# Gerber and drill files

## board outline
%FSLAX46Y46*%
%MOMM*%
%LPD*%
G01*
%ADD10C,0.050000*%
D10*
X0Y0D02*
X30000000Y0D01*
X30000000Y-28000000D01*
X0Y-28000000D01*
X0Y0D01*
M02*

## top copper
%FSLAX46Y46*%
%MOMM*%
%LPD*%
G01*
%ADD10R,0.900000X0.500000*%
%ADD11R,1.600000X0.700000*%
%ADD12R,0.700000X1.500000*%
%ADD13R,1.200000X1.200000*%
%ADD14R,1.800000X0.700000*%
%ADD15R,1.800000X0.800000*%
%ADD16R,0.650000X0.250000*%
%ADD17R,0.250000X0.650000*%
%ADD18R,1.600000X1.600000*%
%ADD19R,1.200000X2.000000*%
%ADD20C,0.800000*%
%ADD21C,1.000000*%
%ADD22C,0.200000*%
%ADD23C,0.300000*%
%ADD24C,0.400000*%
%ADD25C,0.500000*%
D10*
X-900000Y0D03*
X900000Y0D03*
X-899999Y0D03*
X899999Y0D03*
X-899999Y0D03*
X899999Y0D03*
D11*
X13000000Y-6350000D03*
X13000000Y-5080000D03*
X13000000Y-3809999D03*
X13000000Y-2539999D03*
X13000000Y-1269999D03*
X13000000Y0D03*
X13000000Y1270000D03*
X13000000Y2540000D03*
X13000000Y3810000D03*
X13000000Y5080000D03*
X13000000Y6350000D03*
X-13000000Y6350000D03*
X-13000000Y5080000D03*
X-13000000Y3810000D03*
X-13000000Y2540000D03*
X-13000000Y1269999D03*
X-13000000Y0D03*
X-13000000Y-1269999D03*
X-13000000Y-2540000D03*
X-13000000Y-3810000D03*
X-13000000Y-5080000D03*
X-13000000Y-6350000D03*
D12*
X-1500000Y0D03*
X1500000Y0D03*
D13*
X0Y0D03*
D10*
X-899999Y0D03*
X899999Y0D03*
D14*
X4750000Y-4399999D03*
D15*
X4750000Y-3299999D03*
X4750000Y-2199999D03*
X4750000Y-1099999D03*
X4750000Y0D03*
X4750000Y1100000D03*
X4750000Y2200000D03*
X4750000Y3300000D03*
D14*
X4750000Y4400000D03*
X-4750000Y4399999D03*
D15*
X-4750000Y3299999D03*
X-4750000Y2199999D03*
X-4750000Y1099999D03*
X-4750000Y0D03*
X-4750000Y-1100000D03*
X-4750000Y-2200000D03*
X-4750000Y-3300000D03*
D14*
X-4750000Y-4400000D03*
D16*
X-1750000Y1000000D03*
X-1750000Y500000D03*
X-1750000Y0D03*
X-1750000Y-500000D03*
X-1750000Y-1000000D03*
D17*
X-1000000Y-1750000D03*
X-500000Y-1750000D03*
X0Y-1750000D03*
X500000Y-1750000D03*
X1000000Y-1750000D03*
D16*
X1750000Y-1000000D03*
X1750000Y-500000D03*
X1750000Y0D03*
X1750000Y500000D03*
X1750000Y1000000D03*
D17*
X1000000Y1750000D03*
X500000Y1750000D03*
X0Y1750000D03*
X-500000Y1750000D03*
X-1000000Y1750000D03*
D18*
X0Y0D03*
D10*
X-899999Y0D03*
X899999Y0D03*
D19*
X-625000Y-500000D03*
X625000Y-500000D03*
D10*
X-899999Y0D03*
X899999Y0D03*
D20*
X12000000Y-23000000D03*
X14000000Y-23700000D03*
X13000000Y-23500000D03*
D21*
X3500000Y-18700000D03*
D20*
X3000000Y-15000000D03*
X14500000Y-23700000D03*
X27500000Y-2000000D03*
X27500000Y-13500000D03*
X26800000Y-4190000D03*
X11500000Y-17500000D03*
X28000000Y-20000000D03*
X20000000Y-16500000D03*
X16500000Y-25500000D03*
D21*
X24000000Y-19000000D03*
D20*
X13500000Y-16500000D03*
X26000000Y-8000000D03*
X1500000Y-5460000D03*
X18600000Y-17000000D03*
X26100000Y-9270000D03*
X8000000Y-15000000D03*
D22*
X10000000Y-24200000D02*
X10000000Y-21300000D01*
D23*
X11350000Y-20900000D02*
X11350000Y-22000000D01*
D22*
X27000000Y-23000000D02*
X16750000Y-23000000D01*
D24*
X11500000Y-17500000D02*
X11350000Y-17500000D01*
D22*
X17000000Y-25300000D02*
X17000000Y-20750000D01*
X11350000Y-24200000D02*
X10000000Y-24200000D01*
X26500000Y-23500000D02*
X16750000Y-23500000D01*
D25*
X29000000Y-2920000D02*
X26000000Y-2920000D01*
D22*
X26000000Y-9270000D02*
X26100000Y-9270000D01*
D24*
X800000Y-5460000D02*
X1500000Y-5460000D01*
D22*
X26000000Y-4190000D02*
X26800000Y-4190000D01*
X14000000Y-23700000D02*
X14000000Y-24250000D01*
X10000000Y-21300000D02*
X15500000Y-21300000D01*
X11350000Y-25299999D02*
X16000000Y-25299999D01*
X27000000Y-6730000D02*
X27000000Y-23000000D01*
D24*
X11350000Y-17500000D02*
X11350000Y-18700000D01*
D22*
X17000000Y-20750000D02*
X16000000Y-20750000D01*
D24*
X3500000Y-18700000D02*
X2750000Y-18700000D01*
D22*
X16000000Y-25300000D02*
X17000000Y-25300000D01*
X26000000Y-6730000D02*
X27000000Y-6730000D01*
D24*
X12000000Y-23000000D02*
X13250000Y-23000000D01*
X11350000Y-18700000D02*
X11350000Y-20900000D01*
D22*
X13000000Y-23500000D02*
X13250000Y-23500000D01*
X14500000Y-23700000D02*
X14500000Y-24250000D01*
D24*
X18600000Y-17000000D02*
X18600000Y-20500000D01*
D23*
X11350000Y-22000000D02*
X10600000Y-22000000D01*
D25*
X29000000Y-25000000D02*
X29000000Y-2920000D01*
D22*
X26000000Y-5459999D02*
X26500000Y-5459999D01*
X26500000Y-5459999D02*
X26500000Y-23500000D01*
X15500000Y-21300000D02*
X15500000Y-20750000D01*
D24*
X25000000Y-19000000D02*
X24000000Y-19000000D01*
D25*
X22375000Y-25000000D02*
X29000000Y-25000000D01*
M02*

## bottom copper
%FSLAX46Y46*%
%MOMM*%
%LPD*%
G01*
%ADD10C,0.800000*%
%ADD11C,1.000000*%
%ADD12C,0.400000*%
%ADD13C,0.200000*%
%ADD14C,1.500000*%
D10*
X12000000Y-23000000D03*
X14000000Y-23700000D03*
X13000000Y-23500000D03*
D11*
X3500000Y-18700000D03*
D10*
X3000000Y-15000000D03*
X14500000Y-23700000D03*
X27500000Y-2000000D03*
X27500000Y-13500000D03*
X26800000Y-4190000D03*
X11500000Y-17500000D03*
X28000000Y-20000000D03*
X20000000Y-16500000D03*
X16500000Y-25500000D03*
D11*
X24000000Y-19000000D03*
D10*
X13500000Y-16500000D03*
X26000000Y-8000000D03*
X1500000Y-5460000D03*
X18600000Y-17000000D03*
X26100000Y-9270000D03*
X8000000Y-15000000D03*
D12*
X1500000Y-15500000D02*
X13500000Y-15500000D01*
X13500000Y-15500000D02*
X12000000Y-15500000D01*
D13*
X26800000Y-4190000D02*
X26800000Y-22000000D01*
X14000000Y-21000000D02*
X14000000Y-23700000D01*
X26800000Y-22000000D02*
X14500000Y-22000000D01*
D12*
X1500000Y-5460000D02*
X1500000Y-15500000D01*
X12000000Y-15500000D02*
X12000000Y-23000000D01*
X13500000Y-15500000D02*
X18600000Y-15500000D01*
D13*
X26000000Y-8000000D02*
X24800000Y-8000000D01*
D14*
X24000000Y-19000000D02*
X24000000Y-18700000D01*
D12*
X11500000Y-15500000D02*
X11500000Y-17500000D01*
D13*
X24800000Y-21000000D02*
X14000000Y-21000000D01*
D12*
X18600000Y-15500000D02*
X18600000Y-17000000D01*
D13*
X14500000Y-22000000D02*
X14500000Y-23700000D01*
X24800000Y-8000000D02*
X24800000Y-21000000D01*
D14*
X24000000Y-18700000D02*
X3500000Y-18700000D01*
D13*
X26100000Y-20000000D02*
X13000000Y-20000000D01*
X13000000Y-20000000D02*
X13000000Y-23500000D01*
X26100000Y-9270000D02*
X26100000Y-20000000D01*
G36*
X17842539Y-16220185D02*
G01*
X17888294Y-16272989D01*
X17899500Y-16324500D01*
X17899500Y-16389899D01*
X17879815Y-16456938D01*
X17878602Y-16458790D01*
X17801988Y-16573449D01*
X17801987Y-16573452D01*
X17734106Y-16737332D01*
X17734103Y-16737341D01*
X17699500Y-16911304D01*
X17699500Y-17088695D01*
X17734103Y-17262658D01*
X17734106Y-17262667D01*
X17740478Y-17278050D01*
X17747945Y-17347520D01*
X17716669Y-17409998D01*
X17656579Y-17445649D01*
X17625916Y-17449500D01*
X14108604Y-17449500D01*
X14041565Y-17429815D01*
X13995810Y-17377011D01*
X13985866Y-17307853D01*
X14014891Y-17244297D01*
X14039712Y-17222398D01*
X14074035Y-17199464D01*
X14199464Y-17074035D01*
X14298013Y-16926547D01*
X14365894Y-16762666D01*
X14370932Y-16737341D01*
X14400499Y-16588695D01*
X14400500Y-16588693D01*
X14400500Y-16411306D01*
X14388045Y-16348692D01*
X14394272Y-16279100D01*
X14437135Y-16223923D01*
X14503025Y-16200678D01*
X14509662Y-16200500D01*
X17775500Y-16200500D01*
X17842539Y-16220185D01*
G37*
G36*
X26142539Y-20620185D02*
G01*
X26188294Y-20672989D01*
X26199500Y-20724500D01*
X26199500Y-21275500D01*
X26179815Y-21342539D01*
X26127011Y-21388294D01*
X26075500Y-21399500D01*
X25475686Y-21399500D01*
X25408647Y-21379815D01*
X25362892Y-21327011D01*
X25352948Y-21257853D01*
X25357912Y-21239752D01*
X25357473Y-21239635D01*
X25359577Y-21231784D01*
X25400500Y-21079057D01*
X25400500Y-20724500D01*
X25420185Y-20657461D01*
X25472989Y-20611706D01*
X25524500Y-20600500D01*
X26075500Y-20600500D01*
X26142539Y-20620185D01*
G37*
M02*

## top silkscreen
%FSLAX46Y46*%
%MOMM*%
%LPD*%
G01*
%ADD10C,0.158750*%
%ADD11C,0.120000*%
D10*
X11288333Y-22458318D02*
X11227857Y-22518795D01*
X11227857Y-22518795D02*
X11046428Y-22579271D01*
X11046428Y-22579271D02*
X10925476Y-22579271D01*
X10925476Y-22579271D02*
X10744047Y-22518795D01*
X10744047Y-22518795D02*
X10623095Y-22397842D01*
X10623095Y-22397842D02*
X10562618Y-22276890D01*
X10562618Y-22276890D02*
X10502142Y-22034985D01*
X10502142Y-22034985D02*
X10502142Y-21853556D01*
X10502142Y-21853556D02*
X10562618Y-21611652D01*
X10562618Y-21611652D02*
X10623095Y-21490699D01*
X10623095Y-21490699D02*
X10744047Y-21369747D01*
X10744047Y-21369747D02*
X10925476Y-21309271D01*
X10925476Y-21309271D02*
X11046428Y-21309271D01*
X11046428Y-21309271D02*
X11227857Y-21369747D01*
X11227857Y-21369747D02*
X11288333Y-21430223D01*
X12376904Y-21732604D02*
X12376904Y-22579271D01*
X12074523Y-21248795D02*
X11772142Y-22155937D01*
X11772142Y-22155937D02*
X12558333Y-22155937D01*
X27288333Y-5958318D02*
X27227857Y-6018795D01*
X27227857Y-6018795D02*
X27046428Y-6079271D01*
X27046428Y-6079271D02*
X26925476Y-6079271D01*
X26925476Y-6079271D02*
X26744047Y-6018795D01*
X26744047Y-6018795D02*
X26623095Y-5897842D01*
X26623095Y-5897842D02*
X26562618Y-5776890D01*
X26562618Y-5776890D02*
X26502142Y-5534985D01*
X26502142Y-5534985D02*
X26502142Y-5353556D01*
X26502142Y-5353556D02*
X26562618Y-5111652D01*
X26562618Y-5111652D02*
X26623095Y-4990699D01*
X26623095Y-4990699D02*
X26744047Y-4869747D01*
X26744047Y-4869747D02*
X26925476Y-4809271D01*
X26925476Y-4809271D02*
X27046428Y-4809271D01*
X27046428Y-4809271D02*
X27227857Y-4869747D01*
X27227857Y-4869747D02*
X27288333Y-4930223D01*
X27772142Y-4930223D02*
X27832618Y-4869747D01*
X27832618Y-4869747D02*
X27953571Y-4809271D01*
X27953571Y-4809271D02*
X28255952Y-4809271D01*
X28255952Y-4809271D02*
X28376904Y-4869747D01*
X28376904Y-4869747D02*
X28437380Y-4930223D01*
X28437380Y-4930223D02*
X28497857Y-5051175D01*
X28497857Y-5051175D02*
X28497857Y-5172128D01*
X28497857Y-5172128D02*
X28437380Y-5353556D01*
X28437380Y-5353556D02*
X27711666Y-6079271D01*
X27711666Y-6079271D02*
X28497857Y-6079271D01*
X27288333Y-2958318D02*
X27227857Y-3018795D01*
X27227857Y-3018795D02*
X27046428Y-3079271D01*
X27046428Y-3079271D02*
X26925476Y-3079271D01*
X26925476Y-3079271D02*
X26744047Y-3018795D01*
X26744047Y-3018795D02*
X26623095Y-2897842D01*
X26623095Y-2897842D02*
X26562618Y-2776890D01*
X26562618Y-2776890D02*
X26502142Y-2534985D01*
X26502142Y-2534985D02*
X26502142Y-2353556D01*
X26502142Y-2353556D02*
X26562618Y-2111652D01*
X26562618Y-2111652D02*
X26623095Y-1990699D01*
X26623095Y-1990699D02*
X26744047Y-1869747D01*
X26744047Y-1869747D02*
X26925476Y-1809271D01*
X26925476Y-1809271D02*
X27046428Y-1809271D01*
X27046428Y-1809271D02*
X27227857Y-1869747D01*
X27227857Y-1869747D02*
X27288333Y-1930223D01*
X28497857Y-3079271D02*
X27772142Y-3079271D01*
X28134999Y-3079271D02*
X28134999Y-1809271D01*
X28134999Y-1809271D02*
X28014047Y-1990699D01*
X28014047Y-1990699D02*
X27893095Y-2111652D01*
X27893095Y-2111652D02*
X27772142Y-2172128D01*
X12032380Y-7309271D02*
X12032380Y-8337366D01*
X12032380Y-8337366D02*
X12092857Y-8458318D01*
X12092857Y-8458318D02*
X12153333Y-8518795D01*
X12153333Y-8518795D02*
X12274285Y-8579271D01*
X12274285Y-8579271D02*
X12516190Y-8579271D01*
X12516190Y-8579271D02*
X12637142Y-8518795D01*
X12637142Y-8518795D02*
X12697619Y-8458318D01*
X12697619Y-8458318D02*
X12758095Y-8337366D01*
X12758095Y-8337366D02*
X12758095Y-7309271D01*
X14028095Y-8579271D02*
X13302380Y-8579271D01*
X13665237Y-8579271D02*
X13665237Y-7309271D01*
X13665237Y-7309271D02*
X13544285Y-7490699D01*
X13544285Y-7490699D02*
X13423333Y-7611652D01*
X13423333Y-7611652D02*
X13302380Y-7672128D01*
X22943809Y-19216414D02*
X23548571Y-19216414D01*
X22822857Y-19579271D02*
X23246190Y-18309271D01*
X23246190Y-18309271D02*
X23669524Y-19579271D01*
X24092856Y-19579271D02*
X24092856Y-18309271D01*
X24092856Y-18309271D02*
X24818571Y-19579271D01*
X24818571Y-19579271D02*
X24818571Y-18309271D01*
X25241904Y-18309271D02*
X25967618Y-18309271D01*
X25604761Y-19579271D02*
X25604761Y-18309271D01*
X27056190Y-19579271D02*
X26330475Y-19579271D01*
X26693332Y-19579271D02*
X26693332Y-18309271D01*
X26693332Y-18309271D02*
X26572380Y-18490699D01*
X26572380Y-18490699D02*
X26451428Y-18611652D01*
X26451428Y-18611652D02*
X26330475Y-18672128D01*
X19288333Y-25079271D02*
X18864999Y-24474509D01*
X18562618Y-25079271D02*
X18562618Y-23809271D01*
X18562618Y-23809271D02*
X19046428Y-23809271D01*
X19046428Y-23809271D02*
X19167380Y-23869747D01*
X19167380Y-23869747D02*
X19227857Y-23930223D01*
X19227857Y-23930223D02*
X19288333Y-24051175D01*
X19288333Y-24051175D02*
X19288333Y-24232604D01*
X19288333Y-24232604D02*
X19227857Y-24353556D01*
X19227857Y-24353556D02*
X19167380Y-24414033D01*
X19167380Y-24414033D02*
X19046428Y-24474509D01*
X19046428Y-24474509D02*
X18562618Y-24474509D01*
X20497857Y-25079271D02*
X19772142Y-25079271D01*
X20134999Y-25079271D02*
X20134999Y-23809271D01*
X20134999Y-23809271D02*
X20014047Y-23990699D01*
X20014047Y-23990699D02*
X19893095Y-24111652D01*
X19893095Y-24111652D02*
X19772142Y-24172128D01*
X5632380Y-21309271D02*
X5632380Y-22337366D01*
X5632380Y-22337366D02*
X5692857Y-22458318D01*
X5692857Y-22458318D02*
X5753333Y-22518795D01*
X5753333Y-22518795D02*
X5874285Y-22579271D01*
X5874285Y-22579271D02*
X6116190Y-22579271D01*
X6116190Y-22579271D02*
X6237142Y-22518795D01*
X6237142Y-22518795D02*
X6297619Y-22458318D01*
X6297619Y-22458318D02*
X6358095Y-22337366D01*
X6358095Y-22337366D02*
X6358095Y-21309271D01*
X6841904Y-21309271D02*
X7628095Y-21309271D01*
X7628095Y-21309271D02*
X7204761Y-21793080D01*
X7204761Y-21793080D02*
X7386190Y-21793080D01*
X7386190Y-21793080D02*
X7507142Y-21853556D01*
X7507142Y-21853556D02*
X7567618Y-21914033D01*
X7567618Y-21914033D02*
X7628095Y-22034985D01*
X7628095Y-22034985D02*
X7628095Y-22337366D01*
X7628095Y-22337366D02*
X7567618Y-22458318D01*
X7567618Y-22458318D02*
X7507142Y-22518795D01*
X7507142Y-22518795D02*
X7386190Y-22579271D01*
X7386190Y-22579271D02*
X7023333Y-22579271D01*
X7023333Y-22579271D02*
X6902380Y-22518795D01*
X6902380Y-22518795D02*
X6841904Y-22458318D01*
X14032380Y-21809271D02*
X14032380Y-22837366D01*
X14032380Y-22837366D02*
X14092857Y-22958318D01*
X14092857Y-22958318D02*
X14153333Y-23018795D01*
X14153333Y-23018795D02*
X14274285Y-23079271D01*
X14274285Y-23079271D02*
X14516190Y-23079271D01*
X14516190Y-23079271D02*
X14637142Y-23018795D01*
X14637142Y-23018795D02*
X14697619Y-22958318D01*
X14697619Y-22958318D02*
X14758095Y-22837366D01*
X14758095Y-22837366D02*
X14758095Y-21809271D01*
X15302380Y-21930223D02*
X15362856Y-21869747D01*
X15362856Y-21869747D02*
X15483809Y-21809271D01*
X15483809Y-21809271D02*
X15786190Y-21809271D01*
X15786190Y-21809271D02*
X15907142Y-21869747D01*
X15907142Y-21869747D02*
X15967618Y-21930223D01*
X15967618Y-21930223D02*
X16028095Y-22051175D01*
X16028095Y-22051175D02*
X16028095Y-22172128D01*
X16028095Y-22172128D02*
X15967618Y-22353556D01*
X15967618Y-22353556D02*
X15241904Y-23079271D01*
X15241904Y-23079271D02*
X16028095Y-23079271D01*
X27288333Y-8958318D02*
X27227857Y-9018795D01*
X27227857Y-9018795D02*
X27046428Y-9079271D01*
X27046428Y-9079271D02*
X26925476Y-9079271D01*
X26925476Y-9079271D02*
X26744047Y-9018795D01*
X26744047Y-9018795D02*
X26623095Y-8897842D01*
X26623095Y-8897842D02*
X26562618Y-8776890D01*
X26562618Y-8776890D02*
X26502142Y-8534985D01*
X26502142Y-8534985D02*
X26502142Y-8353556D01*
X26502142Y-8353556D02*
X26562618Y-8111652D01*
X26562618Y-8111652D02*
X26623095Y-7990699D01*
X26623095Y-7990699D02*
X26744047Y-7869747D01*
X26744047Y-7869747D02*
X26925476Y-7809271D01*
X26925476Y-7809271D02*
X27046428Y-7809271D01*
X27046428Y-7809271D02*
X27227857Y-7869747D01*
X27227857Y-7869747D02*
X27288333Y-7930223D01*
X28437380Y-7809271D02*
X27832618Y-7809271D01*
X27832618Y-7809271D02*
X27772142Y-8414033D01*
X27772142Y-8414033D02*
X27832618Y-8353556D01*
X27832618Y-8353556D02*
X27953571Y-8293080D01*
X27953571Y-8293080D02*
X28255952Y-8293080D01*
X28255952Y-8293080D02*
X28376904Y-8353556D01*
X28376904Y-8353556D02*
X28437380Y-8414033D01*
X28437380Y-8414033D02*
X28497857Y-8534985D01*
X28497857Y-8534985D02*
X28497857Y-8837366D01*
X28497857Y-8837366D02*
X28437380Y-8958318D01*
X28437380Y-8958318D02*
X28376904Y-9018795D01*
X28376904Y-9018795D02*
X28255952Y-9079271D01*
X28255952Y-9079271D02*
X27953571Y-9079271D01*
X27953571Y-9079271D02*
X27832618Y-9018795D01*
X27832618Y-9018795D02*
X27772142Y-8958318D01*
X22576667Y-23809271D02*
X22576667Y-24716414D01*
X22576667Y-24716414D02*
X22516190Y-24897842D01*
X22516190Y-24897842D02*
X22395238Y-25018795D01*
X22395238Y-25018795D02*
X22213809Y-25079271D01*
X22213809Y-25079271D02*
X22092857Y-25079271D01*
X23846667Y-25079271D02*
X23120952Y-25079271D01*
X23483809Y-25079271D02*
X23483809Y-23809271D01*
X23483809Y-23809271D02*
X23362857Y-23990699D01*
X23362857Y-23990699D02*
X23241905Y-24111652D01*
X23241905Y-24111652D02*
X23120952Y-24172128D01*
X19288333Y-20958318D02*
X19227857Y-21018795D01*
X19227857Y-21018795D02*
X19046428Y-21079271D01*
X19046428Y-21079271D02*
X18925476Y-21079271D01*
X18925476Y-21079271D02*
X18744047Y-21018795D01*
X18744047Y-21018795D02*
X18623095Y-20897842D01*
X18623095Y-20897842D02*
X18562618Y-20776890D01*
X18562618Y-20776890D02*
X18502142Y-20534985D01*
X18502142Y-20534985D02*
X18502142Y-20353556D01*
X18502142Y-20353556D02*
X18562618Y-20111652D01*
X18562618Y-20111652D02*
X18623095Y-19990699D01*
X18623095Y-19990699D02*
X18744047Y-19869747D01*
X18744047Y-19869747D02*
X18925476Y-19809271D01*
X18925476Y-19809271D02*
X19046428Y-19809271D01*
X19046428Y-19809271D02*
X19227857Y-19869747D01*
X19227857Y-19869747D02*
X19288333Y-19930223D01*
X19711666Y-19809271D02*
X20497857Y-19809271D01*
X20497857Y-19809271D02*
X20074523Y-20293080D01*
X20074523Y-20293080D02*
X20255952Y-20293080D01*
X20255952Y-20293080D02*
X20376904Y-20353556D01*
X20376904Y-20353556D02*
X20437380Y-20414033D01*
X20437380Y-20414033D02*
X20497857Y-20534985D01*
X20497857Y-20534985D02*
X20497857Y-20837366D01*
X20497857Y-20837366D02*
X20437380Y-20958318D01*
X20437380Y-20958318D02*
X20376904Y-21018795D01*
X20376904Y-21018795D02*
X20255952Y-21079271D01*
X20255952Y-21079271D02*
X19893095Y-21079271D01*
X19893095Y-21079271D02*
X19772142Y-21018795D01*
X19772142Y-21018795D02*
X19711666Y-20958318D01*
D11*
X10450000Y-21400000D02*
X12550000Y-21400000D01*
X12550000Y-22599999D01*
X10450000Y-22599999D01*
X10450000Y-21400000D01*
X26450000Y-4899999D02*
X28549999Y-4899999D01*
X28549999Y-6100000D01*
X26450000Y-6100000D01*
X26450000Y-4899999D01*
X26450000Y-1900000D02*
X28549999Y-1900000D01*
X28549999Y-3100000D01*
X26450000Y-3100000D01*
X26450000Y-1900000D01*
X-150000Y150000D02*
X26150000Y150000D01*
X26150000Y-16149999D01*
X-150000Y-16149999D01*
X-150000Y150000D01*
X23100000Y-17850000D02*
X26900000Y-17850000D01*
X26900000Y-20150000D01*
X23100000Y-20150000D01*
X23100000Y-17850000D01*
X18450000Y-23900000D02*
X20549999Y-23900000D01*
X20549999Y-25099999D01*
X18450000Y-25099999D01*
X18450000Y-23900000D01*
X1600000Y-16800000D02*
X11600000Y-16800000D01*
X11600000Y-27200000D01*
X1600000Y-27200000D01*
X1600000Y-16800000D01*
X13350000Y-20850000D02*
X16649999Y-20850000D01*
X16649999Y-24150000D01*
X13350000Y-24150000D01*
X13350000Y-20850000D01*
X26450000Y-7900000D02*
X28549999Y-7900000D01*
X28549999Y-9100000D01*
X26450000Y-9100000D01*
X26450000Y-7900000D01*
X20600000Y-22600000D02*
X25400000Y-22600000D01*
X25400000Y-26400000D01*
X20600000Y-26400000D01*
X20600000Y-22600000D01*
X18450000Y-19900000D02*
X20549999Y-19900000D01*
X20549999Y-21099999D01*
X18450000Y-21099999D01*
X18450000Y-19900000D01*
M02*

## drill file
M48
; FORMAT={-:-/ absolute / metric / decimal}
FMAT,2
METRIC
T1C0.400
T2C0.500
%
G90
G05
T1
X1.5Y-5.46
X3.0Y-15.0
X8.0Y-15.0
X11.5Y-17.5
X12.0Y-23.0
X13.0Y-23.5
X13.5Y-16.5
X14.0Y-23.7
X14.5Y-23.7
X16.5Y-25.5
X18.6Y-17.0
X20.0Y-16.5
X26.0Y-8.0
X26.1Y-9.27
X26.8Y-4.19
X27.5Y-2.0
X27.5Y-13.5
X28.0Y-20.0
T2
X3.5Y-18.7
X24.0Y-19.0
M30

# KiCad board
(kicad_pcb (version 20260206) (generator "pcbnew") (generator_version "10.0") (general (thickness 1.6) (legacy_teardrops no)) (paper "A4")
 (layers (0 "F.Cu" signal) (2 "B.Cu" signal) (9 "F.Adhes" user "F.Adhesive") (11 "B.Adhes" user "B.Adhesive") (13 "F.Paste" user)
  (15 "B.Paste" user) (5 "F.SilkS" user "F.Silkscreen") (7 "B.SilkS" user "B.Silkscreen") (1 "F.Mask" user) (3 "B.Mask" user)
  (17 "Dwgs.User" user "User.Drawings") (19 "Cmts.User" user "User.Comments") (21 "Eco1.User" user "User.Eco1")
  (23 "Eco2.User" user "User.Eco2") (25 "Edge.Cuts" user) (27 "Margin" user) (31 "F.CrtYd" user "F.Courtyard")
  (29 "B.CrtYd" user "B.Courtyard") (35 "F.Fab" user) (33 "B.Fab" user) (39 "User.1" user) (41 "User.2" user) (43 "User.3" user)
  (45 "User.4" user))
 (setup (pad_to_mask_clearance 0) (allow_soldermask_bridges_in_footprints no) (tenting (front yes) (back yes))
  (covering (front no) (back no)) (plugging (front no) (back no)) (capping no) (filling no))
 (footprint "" (layer "F.Cu") (at 11.5 22)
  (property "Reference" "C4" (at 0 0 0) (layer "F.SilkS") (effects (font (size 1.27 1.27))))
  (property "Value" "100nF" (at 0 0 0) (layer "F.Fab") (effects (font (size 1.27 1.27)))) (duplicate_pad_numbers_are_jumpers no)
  (fp_rect (start -1.05 -0.6) (end 1.05 0.599999) (stroke (width 0.12) (type default)) (fill no) (layer "F.SilkS"))
  (pad "1" smd rect (at -12.4 -22) (size 0.9 0.5) (layers "F.Cu" "F.Mask" "F.Paste") (thermal_bridge_angle 45))
  (pad "2" smd rect (at -10.6 -22) (size 0.9 0.5) (layers "F.Cu" "F.Mask" "F.Paste") (thermal_bridge_angle 45)))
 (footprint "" (layer "F.Cu") (at 27.5 5.5)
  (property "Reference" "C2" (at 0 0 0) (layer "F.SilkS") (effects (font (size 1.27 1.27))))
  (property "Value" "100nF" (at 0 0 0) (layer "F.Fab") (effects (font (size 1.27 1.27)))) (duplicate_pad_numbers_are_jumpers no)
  (fp_rect (start -1.05 -0.600001) (end 1.049999 0.6) (stroke (width 0.12) (type default)) (fill no) (layer "F.SilkS"))
  (pad "1" smd rect (at -28.399999 -5.5) (size 0.9 0.5) (layers "F.Cu" "F.Mask" "F.Paste") (thermal_bridge_angle 45))
  (pad "2" smd rect (at -26.600001 -5.5) (size 0.9 0.5) (layers "F.Cu" "F.Mask" "F.Paste") (thermal_bridge_angle 45)))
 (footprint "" (layer "F.Cu") (at 27.5 2.5)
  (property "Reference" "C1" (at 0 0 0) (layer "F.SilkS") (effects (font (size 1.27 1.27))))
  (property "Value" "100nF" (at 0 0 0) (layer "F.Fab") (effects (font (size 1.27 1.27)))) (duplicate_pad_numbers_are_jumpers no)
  (fp_rect (start -1.05 -0.6) (end 1.049999 0.6) (stroke (width 0.12) (type default)) (fill no) (layer "F.SilkS"))
  (pad "1" smd rect (at -28.399999 -2.5) (size 0.9 0.5) (layers "F.Cu" "F.Mask" "F.Paste") (thermal_bridge_angle 45))
  (pad "2" smd rect (at -26.600001 -2.5) (size 0.9 0.5) (layers "F.Cu" "F.Mask" "F.Paste") (thermal_bridge_angle 45)))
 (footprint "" (layer "F.Cu") (at 13 8)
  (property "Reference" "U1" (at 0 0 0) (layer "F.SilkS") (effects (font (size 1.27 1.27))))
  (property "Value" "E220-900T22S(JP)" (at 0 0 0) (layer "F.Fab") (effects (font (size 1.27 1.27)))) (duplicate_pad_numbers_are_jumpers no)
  (fp_rect (start -13.15 -8.15) (end 13.15 8.149999) (stroke (width 0.12) (type default)) (fill no) (layer "F.SilkS"))
  (pad "1" smd rect (at 0 -1.65) (size 1.6 0.7) (layers "F.Cu" "F.Mask" "F.Paste") (thermal_bridge_angle 45))
  (pad "2" smd rect (at 0 -2.92) (size 1.6 0.7) (layers "F.Cu" "F.Mask" "F.Paste") (thermal_bridge_angle 45))
  (pad "3" smd rect (at 0 -4.190001) (size 1.6 0.7) (layers "F.Cu" "F.Mask" "F.Paste") (thermal_bridge_angle 45))
  (pad "4" smd rect (at 0 -5.460001) (size 1.6 0.7) (layers "F.Cu" "F.Mask" "F.Paste") (thermal_bridge_angle 45))
  (pad "5" smd rect (at 0 -6.730001) (size 1.6 0.7) (layers "F.Cu" "F.Mask" "F.Paste") (thermal_bridge_angle 45))
  (pad "6" smd rect (at 0 -8) (size 1.6 0.7) (layers "F.Cu" "F.Mask" "F.Paste") (thermal_bridge_angle 45))
  (pad "7" smd rect (at 0 -9.27) (size 1.6 0.7) (layers "F.Cu" "F.Mask" "F.Paste") (thermal_bridge_angle 45))
  (pad "8" smd rect (at 0 -10.54) (size 1.6 0.7) (layers "F.Cu" "F.Mask" "F.Paste") (thermal_bridge_angle 45))
  (pad "9" smd rect (at 0 -11.81) (size 1.6 0.7) (layers "F.Cu" "F.Mask" "F.Paste") (thermal_bridge_angle 45))
  (pad "10" smd rect (at 0 -13.08) (size 1.6 0.7) (layers "F.Cu" "F.Mask" "F.Paste") (thermal_bridge_angle 45))
  (pad "11" smd rect (at 0 -14.35) (size 1.6 0.7) (layers "F.Cu" "F.Mask" "F.Paste") (thermal_bridge_angle 45))
  (pad "12" smd rect (at -26 -14.35) (size 1.6 0.7) (layers "F.Cu" "F.Mask" "F.Paste") (thermal_bridge_angle 45))
  (pad "13" smd rect (at -26 -13.08) (size 1.6 0.7) (layers "F.Cu" "F.Mask" "F.Paste") (thermal_bridge_angle 45))
  (pad "14" smd rect (at -26 -11.81) (size 1.6 0.7) (layers "F.Cu" "F.Mask" "F.Paste") (thermal_bridge_angle 45))
  (pad "15" smd rect (at -26 -10.54) (size 1.6 0.7) (layers "F.Cu" "F.Mask" "F.Paste") (thermal_bridge_angle 45))
  (pad "16" smd rect (at -26 -9.269999) (size 1.6 0.7) (layers "F.Cu" "F.Mask" "F.Paste") (thermal_bridge_angle 45))
  (pad "17" smd rect (at -26 -8) (size 1.6 0.7) (layers "F.Cu" "F.Mask" "F.Paste") (thermal_bridge_angle 45))
  (pad "18" smd rect (at -26 -6.730001) (size 1.6 0.7) (layers "F.Cu" "F.Mask" "F.Paste") (thermal_bridge_angle 45))
  (pad "19" smd rect (at -26 -5.46) (size 1.6 0.7) (layers "F.Cu" "F.Mask" "F.Paste") (thermal_bridge_angle 45))
  (pad "20" smd rect (at -26 -4.19) (size 1.6 0.7) (layers "F.Cu" "F.Mask" "F.Paste") (thermal_bridge_angle 45))
  (pad "21" smd rect (at -26 -2.92) (size 1.6 0.7) (layers "F.Cu" "F.Mask" "F.Paste") (thermal_bridge_angle 45))
  (pad "22" smd rect (at -26 -1.65) (size 1.6 0.7) (layers "F.Cu" "F.Mask" "F.Paste") (thermal_bridge_angle 45)))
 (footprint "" (layer "F.Cu") (at 25 19)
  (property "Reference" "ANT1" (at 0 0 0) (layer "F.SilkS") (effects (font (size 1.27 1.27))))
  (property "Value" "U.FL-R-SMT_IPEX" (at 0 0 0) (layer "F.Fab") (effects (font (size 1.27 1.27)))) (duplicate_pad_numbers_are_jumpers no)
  (fp_rect (start -1.9 -1.15) (end 1.9 1.15) (stroke (width 0.12) (type default)) (fill no) (layer "F.SilkS"))
  (pad "G1" smd rect (at -26.5 -19) (size 0.7 1.5) (layers "F.Cu" "F.Mask" "F.Paste") (thermal_bridge_angle 45))
  (pad "G2" smd rect (at -23.5 -19) (size 0.7 1.5) (layers "F.Cu" "F.Mask" "F.Paste") (thermal_bridge_angle 45))
  (pad "S" smd rect (at -25 -19) (size 1.2 1.2) (layers "F.Cu" "F.Mask" "F.Paste") (thermal_bridge_angle 45)))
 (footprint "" (layer "F.Cu") (at 19.5 24.5)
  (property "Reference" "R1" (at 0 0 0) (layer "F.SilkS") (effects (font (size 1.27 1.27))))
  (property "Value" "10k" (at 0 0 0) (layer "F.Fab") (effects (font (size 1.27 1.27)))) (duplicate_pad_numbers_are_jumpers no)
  (fp_rect (start -1.05 -0.6) (end 1.049999 0.599999) (stroke (width 0.12) (type default)) (fill no) (layer "F.SilkS"))
  (pad "1" smd rect (at -20.399999 -24.5) (size 0.9 0.5) (layers "F.Cu" "F.Mask" "F.Paste") (thermal_bridge_angle 45))
  (pad "2" smd rect (at -18.600001 -24.5) (size 0.9 0.5) (layers "F.Cu" "F.Mask" "F.Paste") (thermal_bridge_angle 45)))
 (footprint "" (layer "F.Cu") (at 6.6 22)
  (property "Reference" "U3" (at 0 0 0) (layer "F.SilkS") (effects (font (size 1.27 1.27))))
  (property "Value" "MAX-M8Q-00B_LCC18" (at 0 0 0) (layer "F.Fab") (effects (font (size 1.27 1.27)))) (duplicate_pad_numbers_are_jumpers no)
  (fp_rect (start -5 -5.2) (end 5 5.2) (stroke (width 0.12) (type default)) (fill no) (layer "F.SilkS"))
  (pad "1" smd rect (at -1.85 -17.600001) (size 1.8 0.7) (layers "F.Cu" "F.Mask" "F.Paste") (thermal_bridge_angle 45))
  (pad "2" smd rect (at -1.85 -18.700001) (size 1.8 0.8) (layers "F.Cu" "F.Mask" "F.Paste") (thermal_bridge_angle 45))
  (pad "3" smd rect (at -1.85 -19.800001) (size 1.8 0.8) (layers "F.Cu" "F.Mask" "F.Paste") (thermal_bridge_angle 45))
  (pad "4" smd rect (at -1.85 -20.900001) (size 1.8 0.8) (layers "F.Cu" "F.Mask" "F.Paste") (thermal_bridge_angle 45))
  (pad "5" smd rect (at -1.85 -22) (size 1.8 0.8) (layers "F.Cu" "F.Mask" "F.Paste") (thermal_bridge_angle 45))
  (pad "6" smd rect (at -1.85 -23.1) (size 1.8 0.8) (layers "F.Cu" "F.Mask" "F.Paste") (thermal_bridge_angle 45))
  (pad "7" smd rect (at -1.85 -24.2) (size 1.8 0.8) (layers "F.Cu" "F.Mask" "F.Paste") (thermal_bridge_angle 45))
  (pad "8" smd rect (at -1.85 -25.3) (size 1.8 0.8) (layers "F.Cu" "F.Mask" "F.Paste") (thermal_bridge_angle 45))
  (pad "9" smd rect (at -1.85 -26.4) (size 1.8 0.7) (layers "F.Cu" "F.Mask" "F.Paste") (thermal_bridge_angle 45))
  (pad "10" smd rect (at -11.35 -26.399999) (size 1.8 0.7) (layers "F.Cu" "F.Mask" "F.Paste") (thermal_bridge_angle 45))
  (pad "11" smd rect (at -11.35 -25.299999) (size 1.8 0.8) (layers "F.Cu" "F.Mask" "F.Paste") (thermal_bridge_angle 45))
  (pad "12" smd rect (at -11.35 -24.199999) (size 1.8 0.8) (layers "F.Cu" "F.Mask" "F.Paste") (thermal_bridge_angle 45))
  (pad "13" smd rect (at -11.35 -23.099999) (size 1.8 0.8) (layers "F.Cu" "F.Mask" "F.Paste") (thermal_bridge_angle 45))
  (pad "14" smd rect (at -11.35 -22) (size 1.8 0.8) (layers "F.Cu" "F.Mask" "F.Paste") (thermal_bridge_angle 45))
  (pad "15" smd rect (at -11.35 -20.9) (size 1.8 0.8) (layers "F.Cu" "F.Mask" "F.Paste") (thermal_bridge_angle 45))
  (pad "16" smd rect (at -11.35 -19.8) (size 1.8 0.8) (layers "F.Cu" "F.Mask" "F.Paste") (thermal_bridge_angle 45))
  (pad "17" smd rect (at -11.35 -18.7) (size 1.8 0.8) (layers "F.Cu" "F.Mask" "F.Paste") (thermal_bridge_angle 45))
  (pad "18" smd rect (at -11.35 -17.6) (size 1.8 0.7) (layers "F.Cu" "F.Mask" "F.Paste") (thermal_bridge_angle 45)))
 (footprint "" (layer "F.Cu") (at 15 22.5)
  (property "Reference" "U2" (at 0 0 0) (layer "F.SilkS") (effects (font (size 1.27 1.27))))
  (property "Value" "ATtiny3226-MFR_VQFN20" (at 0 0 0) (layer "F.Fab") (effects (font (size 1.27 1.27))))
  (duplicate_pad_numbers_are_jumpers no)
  (fp_rect (start -1.65 -1.65) (end 1.649999 1.65) (stroke (width 0.12) (type default)) (fill no) (layer "F.SilkS"))
  (pad "1" smd rect (at -16.75 -23.5) (size 0.65 0.25) (layers "F.Cu" "F.Mask" "F.Paste") (thermal_bridge_angle 45))
  (pad "2" smd rect (at -16.75 -23) (size 0.65 0.25) (layers "F.Cu" "F.Mask" "F.Paste") (thermal_bridge_angle 45))
  (pad "3" smd rect (at -16.75 -22.5) (size 0.65 0.25) (layers "F.Cu" "F.Mask" "F.Paste") (thermal_bridge_angle 45))
  (pad "4" smd rect (at -16.75 -22) (size 0.65 0.25) (layers "F.Cu" "F.Mask" "F.Paste") (thermal_bridge_angle 45))
  (pad "5" smd rect (at -16.75 -21.5) (size 0.65 0.25) (layers "F.Cu" "F.Mask" "F.Paste") (thermal_bridge_angle 45))
  (pad "6" smd rect (at -16 -20.75) (size 0.25 0.65) (layers "F.Cu" "F.Mask" "F.Paste") (thermal_bridge_angle 45))
  (pad "7" smd rect (at -15.5 -20.75) (size 0.25 0.65) (layers "F.Cu" "F.Mask" "F.Paste") (thermal_bridge_angle 45))
  (pad "8" smd rect (at -15 -20.75) (size 0.25 0.65) (layers "F.Cu" "F.Mask" "F.Paste") (thermal_bridge_angle 45))
  (pad "9" smd rect (at -14.5 -20.75) (size 0.25 0.65) (layers "F.Cu" "F.Mask" "F.Paste") (thermal_bridge_angle 45))
  (pad "10" smd rect (at -14 -20.75) (size 0.25 0.65) (layers "F.Cu" "F.Mask" "F.Paste") (thermal_bridge_angle 45))
  (pad "11" smd rect (at -13.25 -21.5) (size 0.65 0.25) (layers "F.Cu" "F.Mask" "F.Paste") (thermal_bridge_angle 45))
  (pad "12" smd rect (at -13.25 -22) (size 0.65 0.25) (layers "F.Cu" "F.Mask" "F.Paste") (thermal_bridge_angle 45))
  (pad "13" smd rect (at -13.25 -22.5) (size 0.65 0.25) (layers "F.Cu" "F.Mask" "F.Paste") (thermal_bridge_angle 45))
  (pad "14" smd rect (at -13.25 -23) (size 0.65 0.25) (layers "F.Cu" "F.Mask" "F.Paste") (thermal_bridge_angle 45))
  (pad "15" smd rect (at -13.25 -23.5) (size 0.65 0.25) (layers "F.Cu" "F.Mask" "F.Paste") (thermal_bridge_angle 45))
  (pad "16" smd rect (at -14 -24.25) (size 0.25 0.65) (layers "F.Cu" "F.Mask" "F.Paste") (thermal_bridge_angle 45))
  (pad "17" smd rect (at -14.5 -24.25) (size 0.25 0.65) (layers "F.Cu" "F.Mask" "F.Paste") (thermal_bridge_angle 45))
  (pad "18" smd rect (at -15 -24.25) (size 0.25 0.65) (layers "F.Cu" "F.Mask" "F.Paste") (thermal_bridge_angle 45))
  (pad "19" smd rect (at -15.5 -24.25) (size 0.25 0.65) (layers "F.Cu" "F.Mask" "F.Paste") (thermal_bridge_angle 45))
  (pad "20" smd rect (at -16 -24.25) (size 0.25 0.65) (layers "F.Cu" "F.Mask" "F.Paste") (thermal_bridge_angle 45))
  (pad "EP" smd rect (at -15 -22.5) (size 1.6 1.6) (layers "F.Cu" "F.Mask" "F.Paste") (thermal_bridge_angle 45)))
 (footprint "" (layer "F.Cu") (at 27.5 8.5)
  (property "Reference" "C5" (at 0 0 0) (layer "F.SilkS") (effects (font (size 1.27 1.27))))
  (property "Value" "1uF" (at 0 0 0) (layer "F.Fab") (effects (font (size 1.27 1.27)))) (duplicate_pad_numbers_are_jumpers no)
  (fp_rect (start -1.05 -0.6) (end 1.049999 0.6) (stroke (width 0.12) (type default)) (fill no) (layer "F.SilkS"))
  (pad "1" smd rect (at -28.399999 -8.5) (size 0.9 0.5) (layers "F.Cu" "F.Mask" "F.Paste") (thermal_bridge_angle 45))
  (pad "2" smd rect (at -26.600001 -8.5) (size 0.9 0.5) (layers "F.Cu" "F.Mask" "F.Paste") (thermal_bridge_angle 45)))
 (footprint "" (layer "F.Cu") (at 23 24.5)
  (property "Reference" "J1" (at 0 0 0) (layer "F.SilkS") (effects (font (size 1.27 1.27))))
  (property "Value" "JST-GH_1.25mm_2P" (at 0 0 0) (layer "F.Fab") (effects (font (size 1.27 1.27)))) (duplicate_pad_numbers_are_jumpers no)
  (fp_rect (start -2.4 -1.9) (end 2.4 1.9) (stroke (width 0.12) (type default)) (fill no) (layer "F.SilkS"))
  (pad "1" smd rect (at -23.625 -24) (size 1.2 2) (layers "F.Cu" "F.Mask" "F.Paste") (thermal_bridge_angle 45))
  (pad "2" smd rect (at -22.375 -24) (size 1.2 2) (layers "F.Cu" "F.Mask" "F.Paste") (thermal_bridge_angle 45)))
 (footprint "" (layer "F.Cu") (at 19.5 20.5)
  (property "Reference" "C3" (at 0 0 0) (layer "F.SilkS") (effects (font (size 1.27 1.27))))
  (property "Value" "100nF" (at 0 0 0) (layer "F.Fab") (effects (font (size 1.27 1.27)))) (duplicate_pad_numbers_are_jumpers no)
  (fp_rect (start -1.05 -0.6) (end 1.049999 0.599999) (stroke (width 0.12) (type default)) (fill no) (layer "F.SilkS"))
  (pad "1" smd rect (at -20.399999 -20.5) (size 0.9 0.5) (layers "F.Cu" "F.Mask" "F.Paste") (thermal_bridge_angle 45))
  (pad "2" smd rect (at -18.600001 -20.5) (size 0.9 0.5) (layers "F.Cu" "F.Mask" "F.Paste") (thermal_bridge_angle 45)))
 (gr_rect (start 0 0) (end 30 28) (stroke (width 0.05) (type default)) (fill no) (layer "Edge.Cuts"))
 (segment (start 10 24.2) (end 10 21.3) (width 0.2) (layer "F.Cu") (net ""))
 (segment (start 11.35 20.9) (end 11.35 22) (width 0.3) (layer "F.Cu") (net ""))
 (segment (start 27 23) (end 16.75 23) (width 0.2) (layer "F.Cu") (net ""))
 (segment (start 11.5 17.5) (end 11.35 17.5) (width 0.4) (layer "F.Cu") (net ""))
 (segment (start 17 25.3) (end 17 20.75) (width 0.2) (layer "F.Cu") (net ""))
 (segment (start 11.35 24.2) (end 10 24.2) (width 0.2) (layer "F.Cu") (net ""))
 (segment (start 26.5 23.5) (end 16.75 23.5) (width 0.2) (layer "F.Cu") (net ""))
 (segment (start 29 2.92) (end 26 2.92) (width 0.5) (layer "F.Cu") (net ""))
 (segment (start 26 9.27) (end 26.1 9.27) (width 0.2) (layer "F.Cu") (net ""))
 (segment (start 0.8 5.46) (end 1.5 5.46) (width 0.4) (layer "F.Cu") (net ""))
 (segment (start 26 4.19) (end 26.8 4.19) (width 0.2) (layer "F.Cu") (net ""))
 (segment (start 14 23.7) (end 14 24.25) (width 0.2) (layer "F.Cu") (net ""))
 (segment (start 10 21.3) (end 15.5 21.3) (width 0.2) (layer "F.Cu") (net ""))
 (segment (start 11.35 25.299999) (end 16 25.299999) (width 0.2) (layer "F.Cu") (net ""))
 (segment (start 27 6.73) (end 27 23) (width 0.2) (layer "F.Cu") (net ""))
 (segment (start 11.35 17.5) (end 11.35 18.7) (width 0.4) (layer "F.Cu") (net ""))
 (segment (start 17 20.75) (end 16 20.75) (width 0.2) (layer "F.Cu") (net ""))
 (segment (start 3.5 18.7) (end 2.75 18.7) (width 0.4) (layer "F.Cu") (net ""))
 (segment (start 16 25.3) (end 17 25.3) (width 0.2) (layer "F.Cu") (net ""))
 (segment (start 26 6.73) (end 27 6.73) (width 0.2) (layer "F.Cu") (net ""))
 (segment (start 12 23) (end 13.25 23) (width 0.4) (layer "F.Cu") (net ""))
 (segment (start 11.35 18.7) (end 11.35 20.9) (width 0.4) (layer "F.Cu") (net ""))
 (segment (start 13 23.5) (end 13.25 23.5) (width 0.2) (layer "F.Cu") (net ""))
 (segment (start 14.5 23.7) (end 14.5 24.25) (width 0.2) (layer "F.Cu") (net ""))
 (segment (start 18.6 17) (end 18.6 20.5) (width 0.4) (layer "F.Cu") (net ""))
 (segment (start 11.35 22) (end 10.6 22) (width 0.3) (layer "F.Cu") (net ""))
 (segment (start 29 25) (end 29 2.92) (width 0.5) (layer "F.Cu") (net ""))
 (segment (start 26 5.459999) (end 26.5 5.459999) (width 0.2) (layer "F.Cu") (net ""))
 (segment (start 26.5 5.459999) (end 26.5 23.5) (width 0.2) (layer "F.Cu") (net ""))
 (segment (start 15.5 21.3) (end 15.5 20.75) (width 0.2) (layer "F.Cu") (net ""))
 (segment (start 25 19) (end 24 19) (width 0.4) (layer "F.Cu") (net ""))
 (segment (start 22.375 25) (end 29 25) (width 0.5) (layer "F.Cu") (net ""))
 (via (at 12 23) (size 0.8) (drill 0.4) (layers "F.Cu" "B.Cu") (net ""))
 (via (at 14 23.7) (size 0.8) (drill 0.4) (layers "F.Cu" "B.Cu") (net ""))
 (via (at 13 23.5) (size 0.8) (drill 0.4) (layers "F.Cu" "B.Cu") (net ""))
 (via (at 3.5 18.7) (size 1) (drill 0.5) (layers "F.Cu" "B.Cu") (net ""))
 (via (at 3 15) (size 0.8) (drill 0.4) (layers "F.Cu" "B.Cu") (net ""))
 (via (at 14.5 23.7) (size 0.8) (drill 0.4) (layers "F.Cu" "B.Cu") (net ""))
 (via (at 27.5 2) (size 0.8) (drill 0.4) (layers "F.Cu" "B.Cu") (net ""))
 (via (at 27.5 13.5) (size 0.8) (drill 0.4) (layers "F.Cu" "B.Cu") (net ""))
 (via (at 26.8 4.19) (size 0.8) (drill 0.4) (layers "F.Cu" "B.Cu") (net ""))
 (via (at 11.5 17.5) (size 0.8) (drill 0.4) (layers "F.Cu" "B.Cu") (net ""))
 (via (at 28 20) (size 0.8) (drill 0.4) (layers "F.Cu" "B.Cu") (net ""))
 (via (at 20 16.5) (size 0.8) (drill 0.4) (layers "F.Cu" "B.Cu") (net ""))
 (via (at 16.5 25.5) (size 0.8) (drill 0.4) (layers "F.Cu" "B.Cu") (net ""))
 (via (at 24 19) (size 1) (drill 0.5) (layers "F.Cu" "B.Cu") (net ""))
 (via (at 13.5 16.5) (size 0.8) (drill 0.4) (layers "F.Cu" "B.Cu") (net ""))
 (via (at 26 8) (size 0.8) (drill 0.4) (layers "F.Cu" "B.Cu") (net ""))
 (via (at 1.5 5.46) (size 0.8) (drill 0.4) (layers "F.Cu" "B.Cu") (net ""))
 (via (at 18.6 17) (size 0.8) (drill 0.4) (layers "F.Cu" "B.Cu") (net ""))
 (via (at 26.1 9.27) (size 0.8) (drill 0.4) (layers "F.Cu" "B.Cu") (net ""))
 (via (at 8 15) (size 0.8) (drill 0.4) (layers "F.Cu" "B.Cu") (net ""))
 (segment (start 1.5 15.5) (end 13.5 15.5) (width 0.4) (layer "B.Cu") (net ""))
 (segment (start 13.5 15.5) (end 12 15.5) (width 0.4) (layer "B.Cu") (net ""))
 (segment (start 26.8 4.19) (end 26.8 22) (width 0.2) (layer "B.Cu") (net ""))
 (segment (start 14 21) (end 14 23.7) (width 0.2) (layer "B.Cu") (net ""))
 (segment (start 26.8 22) (end 14.5 22) (width 0.2) (layer "B.Cu") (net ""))
 (segment (start 1.5 5.46) (end 1.5 15.5) (width 0.4) (layer "B.Cu") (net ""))
 (segment (start 12 15.5) (end 12 23) (width 0.4) (layer "B.Cu") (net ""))
 (segment (start 13.5 15.5) (end 18.6 15.5) (width 0.4) (layer "B.Cu") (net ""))
 (segment (start 26 8) (end 24.8 8) (width 0.2) (layer "B.Cu") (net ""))
 (segment (start 24 19) (end 24 18.7) (width 1.5) (layer "B.Cu") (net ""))
 (segment (start 11.5 15.5) (end 11.5 17.5) (width 0.4) (layer "B.Cu") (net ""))
 (segment (start 24.8 21) (end 14 21) (width 0.2) (layer "B.Cu") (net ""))
 (segment (start 18.6 15.5) (end 18.6 17) (width 0.4) (layer "B.Cu") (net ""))
 (segment (start 14.5 22) (end 14.5 23.7) (width 0.2) (layer "B.Cu") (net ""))
 (segment (start 24.8 8) (end 24.8 21) (width 0.2) (layer "B.Cu") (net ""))
 (segment (start 24 18.7) (end 3.5 18.7) (width 1.5) (layer "B.Cu") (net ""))
 (segment (start 26.1 20) (end 13 20) (width 0.2) (layer "B.Cu") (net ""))
 (segment (start 13 20) (end 13 23.5) (width 0.2) (layer "B.Cu") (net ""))
 (segment (start 26.1 9.27) (end 26.1 20) (width 0.2) (layer "B.Cu") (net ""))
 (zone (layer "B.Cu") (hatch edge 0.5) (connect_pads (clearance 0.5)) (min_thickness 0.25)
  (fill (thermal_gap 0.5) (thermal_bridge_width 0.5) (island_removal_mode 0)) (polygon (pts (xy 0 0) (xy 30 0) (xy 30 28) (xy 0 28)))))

